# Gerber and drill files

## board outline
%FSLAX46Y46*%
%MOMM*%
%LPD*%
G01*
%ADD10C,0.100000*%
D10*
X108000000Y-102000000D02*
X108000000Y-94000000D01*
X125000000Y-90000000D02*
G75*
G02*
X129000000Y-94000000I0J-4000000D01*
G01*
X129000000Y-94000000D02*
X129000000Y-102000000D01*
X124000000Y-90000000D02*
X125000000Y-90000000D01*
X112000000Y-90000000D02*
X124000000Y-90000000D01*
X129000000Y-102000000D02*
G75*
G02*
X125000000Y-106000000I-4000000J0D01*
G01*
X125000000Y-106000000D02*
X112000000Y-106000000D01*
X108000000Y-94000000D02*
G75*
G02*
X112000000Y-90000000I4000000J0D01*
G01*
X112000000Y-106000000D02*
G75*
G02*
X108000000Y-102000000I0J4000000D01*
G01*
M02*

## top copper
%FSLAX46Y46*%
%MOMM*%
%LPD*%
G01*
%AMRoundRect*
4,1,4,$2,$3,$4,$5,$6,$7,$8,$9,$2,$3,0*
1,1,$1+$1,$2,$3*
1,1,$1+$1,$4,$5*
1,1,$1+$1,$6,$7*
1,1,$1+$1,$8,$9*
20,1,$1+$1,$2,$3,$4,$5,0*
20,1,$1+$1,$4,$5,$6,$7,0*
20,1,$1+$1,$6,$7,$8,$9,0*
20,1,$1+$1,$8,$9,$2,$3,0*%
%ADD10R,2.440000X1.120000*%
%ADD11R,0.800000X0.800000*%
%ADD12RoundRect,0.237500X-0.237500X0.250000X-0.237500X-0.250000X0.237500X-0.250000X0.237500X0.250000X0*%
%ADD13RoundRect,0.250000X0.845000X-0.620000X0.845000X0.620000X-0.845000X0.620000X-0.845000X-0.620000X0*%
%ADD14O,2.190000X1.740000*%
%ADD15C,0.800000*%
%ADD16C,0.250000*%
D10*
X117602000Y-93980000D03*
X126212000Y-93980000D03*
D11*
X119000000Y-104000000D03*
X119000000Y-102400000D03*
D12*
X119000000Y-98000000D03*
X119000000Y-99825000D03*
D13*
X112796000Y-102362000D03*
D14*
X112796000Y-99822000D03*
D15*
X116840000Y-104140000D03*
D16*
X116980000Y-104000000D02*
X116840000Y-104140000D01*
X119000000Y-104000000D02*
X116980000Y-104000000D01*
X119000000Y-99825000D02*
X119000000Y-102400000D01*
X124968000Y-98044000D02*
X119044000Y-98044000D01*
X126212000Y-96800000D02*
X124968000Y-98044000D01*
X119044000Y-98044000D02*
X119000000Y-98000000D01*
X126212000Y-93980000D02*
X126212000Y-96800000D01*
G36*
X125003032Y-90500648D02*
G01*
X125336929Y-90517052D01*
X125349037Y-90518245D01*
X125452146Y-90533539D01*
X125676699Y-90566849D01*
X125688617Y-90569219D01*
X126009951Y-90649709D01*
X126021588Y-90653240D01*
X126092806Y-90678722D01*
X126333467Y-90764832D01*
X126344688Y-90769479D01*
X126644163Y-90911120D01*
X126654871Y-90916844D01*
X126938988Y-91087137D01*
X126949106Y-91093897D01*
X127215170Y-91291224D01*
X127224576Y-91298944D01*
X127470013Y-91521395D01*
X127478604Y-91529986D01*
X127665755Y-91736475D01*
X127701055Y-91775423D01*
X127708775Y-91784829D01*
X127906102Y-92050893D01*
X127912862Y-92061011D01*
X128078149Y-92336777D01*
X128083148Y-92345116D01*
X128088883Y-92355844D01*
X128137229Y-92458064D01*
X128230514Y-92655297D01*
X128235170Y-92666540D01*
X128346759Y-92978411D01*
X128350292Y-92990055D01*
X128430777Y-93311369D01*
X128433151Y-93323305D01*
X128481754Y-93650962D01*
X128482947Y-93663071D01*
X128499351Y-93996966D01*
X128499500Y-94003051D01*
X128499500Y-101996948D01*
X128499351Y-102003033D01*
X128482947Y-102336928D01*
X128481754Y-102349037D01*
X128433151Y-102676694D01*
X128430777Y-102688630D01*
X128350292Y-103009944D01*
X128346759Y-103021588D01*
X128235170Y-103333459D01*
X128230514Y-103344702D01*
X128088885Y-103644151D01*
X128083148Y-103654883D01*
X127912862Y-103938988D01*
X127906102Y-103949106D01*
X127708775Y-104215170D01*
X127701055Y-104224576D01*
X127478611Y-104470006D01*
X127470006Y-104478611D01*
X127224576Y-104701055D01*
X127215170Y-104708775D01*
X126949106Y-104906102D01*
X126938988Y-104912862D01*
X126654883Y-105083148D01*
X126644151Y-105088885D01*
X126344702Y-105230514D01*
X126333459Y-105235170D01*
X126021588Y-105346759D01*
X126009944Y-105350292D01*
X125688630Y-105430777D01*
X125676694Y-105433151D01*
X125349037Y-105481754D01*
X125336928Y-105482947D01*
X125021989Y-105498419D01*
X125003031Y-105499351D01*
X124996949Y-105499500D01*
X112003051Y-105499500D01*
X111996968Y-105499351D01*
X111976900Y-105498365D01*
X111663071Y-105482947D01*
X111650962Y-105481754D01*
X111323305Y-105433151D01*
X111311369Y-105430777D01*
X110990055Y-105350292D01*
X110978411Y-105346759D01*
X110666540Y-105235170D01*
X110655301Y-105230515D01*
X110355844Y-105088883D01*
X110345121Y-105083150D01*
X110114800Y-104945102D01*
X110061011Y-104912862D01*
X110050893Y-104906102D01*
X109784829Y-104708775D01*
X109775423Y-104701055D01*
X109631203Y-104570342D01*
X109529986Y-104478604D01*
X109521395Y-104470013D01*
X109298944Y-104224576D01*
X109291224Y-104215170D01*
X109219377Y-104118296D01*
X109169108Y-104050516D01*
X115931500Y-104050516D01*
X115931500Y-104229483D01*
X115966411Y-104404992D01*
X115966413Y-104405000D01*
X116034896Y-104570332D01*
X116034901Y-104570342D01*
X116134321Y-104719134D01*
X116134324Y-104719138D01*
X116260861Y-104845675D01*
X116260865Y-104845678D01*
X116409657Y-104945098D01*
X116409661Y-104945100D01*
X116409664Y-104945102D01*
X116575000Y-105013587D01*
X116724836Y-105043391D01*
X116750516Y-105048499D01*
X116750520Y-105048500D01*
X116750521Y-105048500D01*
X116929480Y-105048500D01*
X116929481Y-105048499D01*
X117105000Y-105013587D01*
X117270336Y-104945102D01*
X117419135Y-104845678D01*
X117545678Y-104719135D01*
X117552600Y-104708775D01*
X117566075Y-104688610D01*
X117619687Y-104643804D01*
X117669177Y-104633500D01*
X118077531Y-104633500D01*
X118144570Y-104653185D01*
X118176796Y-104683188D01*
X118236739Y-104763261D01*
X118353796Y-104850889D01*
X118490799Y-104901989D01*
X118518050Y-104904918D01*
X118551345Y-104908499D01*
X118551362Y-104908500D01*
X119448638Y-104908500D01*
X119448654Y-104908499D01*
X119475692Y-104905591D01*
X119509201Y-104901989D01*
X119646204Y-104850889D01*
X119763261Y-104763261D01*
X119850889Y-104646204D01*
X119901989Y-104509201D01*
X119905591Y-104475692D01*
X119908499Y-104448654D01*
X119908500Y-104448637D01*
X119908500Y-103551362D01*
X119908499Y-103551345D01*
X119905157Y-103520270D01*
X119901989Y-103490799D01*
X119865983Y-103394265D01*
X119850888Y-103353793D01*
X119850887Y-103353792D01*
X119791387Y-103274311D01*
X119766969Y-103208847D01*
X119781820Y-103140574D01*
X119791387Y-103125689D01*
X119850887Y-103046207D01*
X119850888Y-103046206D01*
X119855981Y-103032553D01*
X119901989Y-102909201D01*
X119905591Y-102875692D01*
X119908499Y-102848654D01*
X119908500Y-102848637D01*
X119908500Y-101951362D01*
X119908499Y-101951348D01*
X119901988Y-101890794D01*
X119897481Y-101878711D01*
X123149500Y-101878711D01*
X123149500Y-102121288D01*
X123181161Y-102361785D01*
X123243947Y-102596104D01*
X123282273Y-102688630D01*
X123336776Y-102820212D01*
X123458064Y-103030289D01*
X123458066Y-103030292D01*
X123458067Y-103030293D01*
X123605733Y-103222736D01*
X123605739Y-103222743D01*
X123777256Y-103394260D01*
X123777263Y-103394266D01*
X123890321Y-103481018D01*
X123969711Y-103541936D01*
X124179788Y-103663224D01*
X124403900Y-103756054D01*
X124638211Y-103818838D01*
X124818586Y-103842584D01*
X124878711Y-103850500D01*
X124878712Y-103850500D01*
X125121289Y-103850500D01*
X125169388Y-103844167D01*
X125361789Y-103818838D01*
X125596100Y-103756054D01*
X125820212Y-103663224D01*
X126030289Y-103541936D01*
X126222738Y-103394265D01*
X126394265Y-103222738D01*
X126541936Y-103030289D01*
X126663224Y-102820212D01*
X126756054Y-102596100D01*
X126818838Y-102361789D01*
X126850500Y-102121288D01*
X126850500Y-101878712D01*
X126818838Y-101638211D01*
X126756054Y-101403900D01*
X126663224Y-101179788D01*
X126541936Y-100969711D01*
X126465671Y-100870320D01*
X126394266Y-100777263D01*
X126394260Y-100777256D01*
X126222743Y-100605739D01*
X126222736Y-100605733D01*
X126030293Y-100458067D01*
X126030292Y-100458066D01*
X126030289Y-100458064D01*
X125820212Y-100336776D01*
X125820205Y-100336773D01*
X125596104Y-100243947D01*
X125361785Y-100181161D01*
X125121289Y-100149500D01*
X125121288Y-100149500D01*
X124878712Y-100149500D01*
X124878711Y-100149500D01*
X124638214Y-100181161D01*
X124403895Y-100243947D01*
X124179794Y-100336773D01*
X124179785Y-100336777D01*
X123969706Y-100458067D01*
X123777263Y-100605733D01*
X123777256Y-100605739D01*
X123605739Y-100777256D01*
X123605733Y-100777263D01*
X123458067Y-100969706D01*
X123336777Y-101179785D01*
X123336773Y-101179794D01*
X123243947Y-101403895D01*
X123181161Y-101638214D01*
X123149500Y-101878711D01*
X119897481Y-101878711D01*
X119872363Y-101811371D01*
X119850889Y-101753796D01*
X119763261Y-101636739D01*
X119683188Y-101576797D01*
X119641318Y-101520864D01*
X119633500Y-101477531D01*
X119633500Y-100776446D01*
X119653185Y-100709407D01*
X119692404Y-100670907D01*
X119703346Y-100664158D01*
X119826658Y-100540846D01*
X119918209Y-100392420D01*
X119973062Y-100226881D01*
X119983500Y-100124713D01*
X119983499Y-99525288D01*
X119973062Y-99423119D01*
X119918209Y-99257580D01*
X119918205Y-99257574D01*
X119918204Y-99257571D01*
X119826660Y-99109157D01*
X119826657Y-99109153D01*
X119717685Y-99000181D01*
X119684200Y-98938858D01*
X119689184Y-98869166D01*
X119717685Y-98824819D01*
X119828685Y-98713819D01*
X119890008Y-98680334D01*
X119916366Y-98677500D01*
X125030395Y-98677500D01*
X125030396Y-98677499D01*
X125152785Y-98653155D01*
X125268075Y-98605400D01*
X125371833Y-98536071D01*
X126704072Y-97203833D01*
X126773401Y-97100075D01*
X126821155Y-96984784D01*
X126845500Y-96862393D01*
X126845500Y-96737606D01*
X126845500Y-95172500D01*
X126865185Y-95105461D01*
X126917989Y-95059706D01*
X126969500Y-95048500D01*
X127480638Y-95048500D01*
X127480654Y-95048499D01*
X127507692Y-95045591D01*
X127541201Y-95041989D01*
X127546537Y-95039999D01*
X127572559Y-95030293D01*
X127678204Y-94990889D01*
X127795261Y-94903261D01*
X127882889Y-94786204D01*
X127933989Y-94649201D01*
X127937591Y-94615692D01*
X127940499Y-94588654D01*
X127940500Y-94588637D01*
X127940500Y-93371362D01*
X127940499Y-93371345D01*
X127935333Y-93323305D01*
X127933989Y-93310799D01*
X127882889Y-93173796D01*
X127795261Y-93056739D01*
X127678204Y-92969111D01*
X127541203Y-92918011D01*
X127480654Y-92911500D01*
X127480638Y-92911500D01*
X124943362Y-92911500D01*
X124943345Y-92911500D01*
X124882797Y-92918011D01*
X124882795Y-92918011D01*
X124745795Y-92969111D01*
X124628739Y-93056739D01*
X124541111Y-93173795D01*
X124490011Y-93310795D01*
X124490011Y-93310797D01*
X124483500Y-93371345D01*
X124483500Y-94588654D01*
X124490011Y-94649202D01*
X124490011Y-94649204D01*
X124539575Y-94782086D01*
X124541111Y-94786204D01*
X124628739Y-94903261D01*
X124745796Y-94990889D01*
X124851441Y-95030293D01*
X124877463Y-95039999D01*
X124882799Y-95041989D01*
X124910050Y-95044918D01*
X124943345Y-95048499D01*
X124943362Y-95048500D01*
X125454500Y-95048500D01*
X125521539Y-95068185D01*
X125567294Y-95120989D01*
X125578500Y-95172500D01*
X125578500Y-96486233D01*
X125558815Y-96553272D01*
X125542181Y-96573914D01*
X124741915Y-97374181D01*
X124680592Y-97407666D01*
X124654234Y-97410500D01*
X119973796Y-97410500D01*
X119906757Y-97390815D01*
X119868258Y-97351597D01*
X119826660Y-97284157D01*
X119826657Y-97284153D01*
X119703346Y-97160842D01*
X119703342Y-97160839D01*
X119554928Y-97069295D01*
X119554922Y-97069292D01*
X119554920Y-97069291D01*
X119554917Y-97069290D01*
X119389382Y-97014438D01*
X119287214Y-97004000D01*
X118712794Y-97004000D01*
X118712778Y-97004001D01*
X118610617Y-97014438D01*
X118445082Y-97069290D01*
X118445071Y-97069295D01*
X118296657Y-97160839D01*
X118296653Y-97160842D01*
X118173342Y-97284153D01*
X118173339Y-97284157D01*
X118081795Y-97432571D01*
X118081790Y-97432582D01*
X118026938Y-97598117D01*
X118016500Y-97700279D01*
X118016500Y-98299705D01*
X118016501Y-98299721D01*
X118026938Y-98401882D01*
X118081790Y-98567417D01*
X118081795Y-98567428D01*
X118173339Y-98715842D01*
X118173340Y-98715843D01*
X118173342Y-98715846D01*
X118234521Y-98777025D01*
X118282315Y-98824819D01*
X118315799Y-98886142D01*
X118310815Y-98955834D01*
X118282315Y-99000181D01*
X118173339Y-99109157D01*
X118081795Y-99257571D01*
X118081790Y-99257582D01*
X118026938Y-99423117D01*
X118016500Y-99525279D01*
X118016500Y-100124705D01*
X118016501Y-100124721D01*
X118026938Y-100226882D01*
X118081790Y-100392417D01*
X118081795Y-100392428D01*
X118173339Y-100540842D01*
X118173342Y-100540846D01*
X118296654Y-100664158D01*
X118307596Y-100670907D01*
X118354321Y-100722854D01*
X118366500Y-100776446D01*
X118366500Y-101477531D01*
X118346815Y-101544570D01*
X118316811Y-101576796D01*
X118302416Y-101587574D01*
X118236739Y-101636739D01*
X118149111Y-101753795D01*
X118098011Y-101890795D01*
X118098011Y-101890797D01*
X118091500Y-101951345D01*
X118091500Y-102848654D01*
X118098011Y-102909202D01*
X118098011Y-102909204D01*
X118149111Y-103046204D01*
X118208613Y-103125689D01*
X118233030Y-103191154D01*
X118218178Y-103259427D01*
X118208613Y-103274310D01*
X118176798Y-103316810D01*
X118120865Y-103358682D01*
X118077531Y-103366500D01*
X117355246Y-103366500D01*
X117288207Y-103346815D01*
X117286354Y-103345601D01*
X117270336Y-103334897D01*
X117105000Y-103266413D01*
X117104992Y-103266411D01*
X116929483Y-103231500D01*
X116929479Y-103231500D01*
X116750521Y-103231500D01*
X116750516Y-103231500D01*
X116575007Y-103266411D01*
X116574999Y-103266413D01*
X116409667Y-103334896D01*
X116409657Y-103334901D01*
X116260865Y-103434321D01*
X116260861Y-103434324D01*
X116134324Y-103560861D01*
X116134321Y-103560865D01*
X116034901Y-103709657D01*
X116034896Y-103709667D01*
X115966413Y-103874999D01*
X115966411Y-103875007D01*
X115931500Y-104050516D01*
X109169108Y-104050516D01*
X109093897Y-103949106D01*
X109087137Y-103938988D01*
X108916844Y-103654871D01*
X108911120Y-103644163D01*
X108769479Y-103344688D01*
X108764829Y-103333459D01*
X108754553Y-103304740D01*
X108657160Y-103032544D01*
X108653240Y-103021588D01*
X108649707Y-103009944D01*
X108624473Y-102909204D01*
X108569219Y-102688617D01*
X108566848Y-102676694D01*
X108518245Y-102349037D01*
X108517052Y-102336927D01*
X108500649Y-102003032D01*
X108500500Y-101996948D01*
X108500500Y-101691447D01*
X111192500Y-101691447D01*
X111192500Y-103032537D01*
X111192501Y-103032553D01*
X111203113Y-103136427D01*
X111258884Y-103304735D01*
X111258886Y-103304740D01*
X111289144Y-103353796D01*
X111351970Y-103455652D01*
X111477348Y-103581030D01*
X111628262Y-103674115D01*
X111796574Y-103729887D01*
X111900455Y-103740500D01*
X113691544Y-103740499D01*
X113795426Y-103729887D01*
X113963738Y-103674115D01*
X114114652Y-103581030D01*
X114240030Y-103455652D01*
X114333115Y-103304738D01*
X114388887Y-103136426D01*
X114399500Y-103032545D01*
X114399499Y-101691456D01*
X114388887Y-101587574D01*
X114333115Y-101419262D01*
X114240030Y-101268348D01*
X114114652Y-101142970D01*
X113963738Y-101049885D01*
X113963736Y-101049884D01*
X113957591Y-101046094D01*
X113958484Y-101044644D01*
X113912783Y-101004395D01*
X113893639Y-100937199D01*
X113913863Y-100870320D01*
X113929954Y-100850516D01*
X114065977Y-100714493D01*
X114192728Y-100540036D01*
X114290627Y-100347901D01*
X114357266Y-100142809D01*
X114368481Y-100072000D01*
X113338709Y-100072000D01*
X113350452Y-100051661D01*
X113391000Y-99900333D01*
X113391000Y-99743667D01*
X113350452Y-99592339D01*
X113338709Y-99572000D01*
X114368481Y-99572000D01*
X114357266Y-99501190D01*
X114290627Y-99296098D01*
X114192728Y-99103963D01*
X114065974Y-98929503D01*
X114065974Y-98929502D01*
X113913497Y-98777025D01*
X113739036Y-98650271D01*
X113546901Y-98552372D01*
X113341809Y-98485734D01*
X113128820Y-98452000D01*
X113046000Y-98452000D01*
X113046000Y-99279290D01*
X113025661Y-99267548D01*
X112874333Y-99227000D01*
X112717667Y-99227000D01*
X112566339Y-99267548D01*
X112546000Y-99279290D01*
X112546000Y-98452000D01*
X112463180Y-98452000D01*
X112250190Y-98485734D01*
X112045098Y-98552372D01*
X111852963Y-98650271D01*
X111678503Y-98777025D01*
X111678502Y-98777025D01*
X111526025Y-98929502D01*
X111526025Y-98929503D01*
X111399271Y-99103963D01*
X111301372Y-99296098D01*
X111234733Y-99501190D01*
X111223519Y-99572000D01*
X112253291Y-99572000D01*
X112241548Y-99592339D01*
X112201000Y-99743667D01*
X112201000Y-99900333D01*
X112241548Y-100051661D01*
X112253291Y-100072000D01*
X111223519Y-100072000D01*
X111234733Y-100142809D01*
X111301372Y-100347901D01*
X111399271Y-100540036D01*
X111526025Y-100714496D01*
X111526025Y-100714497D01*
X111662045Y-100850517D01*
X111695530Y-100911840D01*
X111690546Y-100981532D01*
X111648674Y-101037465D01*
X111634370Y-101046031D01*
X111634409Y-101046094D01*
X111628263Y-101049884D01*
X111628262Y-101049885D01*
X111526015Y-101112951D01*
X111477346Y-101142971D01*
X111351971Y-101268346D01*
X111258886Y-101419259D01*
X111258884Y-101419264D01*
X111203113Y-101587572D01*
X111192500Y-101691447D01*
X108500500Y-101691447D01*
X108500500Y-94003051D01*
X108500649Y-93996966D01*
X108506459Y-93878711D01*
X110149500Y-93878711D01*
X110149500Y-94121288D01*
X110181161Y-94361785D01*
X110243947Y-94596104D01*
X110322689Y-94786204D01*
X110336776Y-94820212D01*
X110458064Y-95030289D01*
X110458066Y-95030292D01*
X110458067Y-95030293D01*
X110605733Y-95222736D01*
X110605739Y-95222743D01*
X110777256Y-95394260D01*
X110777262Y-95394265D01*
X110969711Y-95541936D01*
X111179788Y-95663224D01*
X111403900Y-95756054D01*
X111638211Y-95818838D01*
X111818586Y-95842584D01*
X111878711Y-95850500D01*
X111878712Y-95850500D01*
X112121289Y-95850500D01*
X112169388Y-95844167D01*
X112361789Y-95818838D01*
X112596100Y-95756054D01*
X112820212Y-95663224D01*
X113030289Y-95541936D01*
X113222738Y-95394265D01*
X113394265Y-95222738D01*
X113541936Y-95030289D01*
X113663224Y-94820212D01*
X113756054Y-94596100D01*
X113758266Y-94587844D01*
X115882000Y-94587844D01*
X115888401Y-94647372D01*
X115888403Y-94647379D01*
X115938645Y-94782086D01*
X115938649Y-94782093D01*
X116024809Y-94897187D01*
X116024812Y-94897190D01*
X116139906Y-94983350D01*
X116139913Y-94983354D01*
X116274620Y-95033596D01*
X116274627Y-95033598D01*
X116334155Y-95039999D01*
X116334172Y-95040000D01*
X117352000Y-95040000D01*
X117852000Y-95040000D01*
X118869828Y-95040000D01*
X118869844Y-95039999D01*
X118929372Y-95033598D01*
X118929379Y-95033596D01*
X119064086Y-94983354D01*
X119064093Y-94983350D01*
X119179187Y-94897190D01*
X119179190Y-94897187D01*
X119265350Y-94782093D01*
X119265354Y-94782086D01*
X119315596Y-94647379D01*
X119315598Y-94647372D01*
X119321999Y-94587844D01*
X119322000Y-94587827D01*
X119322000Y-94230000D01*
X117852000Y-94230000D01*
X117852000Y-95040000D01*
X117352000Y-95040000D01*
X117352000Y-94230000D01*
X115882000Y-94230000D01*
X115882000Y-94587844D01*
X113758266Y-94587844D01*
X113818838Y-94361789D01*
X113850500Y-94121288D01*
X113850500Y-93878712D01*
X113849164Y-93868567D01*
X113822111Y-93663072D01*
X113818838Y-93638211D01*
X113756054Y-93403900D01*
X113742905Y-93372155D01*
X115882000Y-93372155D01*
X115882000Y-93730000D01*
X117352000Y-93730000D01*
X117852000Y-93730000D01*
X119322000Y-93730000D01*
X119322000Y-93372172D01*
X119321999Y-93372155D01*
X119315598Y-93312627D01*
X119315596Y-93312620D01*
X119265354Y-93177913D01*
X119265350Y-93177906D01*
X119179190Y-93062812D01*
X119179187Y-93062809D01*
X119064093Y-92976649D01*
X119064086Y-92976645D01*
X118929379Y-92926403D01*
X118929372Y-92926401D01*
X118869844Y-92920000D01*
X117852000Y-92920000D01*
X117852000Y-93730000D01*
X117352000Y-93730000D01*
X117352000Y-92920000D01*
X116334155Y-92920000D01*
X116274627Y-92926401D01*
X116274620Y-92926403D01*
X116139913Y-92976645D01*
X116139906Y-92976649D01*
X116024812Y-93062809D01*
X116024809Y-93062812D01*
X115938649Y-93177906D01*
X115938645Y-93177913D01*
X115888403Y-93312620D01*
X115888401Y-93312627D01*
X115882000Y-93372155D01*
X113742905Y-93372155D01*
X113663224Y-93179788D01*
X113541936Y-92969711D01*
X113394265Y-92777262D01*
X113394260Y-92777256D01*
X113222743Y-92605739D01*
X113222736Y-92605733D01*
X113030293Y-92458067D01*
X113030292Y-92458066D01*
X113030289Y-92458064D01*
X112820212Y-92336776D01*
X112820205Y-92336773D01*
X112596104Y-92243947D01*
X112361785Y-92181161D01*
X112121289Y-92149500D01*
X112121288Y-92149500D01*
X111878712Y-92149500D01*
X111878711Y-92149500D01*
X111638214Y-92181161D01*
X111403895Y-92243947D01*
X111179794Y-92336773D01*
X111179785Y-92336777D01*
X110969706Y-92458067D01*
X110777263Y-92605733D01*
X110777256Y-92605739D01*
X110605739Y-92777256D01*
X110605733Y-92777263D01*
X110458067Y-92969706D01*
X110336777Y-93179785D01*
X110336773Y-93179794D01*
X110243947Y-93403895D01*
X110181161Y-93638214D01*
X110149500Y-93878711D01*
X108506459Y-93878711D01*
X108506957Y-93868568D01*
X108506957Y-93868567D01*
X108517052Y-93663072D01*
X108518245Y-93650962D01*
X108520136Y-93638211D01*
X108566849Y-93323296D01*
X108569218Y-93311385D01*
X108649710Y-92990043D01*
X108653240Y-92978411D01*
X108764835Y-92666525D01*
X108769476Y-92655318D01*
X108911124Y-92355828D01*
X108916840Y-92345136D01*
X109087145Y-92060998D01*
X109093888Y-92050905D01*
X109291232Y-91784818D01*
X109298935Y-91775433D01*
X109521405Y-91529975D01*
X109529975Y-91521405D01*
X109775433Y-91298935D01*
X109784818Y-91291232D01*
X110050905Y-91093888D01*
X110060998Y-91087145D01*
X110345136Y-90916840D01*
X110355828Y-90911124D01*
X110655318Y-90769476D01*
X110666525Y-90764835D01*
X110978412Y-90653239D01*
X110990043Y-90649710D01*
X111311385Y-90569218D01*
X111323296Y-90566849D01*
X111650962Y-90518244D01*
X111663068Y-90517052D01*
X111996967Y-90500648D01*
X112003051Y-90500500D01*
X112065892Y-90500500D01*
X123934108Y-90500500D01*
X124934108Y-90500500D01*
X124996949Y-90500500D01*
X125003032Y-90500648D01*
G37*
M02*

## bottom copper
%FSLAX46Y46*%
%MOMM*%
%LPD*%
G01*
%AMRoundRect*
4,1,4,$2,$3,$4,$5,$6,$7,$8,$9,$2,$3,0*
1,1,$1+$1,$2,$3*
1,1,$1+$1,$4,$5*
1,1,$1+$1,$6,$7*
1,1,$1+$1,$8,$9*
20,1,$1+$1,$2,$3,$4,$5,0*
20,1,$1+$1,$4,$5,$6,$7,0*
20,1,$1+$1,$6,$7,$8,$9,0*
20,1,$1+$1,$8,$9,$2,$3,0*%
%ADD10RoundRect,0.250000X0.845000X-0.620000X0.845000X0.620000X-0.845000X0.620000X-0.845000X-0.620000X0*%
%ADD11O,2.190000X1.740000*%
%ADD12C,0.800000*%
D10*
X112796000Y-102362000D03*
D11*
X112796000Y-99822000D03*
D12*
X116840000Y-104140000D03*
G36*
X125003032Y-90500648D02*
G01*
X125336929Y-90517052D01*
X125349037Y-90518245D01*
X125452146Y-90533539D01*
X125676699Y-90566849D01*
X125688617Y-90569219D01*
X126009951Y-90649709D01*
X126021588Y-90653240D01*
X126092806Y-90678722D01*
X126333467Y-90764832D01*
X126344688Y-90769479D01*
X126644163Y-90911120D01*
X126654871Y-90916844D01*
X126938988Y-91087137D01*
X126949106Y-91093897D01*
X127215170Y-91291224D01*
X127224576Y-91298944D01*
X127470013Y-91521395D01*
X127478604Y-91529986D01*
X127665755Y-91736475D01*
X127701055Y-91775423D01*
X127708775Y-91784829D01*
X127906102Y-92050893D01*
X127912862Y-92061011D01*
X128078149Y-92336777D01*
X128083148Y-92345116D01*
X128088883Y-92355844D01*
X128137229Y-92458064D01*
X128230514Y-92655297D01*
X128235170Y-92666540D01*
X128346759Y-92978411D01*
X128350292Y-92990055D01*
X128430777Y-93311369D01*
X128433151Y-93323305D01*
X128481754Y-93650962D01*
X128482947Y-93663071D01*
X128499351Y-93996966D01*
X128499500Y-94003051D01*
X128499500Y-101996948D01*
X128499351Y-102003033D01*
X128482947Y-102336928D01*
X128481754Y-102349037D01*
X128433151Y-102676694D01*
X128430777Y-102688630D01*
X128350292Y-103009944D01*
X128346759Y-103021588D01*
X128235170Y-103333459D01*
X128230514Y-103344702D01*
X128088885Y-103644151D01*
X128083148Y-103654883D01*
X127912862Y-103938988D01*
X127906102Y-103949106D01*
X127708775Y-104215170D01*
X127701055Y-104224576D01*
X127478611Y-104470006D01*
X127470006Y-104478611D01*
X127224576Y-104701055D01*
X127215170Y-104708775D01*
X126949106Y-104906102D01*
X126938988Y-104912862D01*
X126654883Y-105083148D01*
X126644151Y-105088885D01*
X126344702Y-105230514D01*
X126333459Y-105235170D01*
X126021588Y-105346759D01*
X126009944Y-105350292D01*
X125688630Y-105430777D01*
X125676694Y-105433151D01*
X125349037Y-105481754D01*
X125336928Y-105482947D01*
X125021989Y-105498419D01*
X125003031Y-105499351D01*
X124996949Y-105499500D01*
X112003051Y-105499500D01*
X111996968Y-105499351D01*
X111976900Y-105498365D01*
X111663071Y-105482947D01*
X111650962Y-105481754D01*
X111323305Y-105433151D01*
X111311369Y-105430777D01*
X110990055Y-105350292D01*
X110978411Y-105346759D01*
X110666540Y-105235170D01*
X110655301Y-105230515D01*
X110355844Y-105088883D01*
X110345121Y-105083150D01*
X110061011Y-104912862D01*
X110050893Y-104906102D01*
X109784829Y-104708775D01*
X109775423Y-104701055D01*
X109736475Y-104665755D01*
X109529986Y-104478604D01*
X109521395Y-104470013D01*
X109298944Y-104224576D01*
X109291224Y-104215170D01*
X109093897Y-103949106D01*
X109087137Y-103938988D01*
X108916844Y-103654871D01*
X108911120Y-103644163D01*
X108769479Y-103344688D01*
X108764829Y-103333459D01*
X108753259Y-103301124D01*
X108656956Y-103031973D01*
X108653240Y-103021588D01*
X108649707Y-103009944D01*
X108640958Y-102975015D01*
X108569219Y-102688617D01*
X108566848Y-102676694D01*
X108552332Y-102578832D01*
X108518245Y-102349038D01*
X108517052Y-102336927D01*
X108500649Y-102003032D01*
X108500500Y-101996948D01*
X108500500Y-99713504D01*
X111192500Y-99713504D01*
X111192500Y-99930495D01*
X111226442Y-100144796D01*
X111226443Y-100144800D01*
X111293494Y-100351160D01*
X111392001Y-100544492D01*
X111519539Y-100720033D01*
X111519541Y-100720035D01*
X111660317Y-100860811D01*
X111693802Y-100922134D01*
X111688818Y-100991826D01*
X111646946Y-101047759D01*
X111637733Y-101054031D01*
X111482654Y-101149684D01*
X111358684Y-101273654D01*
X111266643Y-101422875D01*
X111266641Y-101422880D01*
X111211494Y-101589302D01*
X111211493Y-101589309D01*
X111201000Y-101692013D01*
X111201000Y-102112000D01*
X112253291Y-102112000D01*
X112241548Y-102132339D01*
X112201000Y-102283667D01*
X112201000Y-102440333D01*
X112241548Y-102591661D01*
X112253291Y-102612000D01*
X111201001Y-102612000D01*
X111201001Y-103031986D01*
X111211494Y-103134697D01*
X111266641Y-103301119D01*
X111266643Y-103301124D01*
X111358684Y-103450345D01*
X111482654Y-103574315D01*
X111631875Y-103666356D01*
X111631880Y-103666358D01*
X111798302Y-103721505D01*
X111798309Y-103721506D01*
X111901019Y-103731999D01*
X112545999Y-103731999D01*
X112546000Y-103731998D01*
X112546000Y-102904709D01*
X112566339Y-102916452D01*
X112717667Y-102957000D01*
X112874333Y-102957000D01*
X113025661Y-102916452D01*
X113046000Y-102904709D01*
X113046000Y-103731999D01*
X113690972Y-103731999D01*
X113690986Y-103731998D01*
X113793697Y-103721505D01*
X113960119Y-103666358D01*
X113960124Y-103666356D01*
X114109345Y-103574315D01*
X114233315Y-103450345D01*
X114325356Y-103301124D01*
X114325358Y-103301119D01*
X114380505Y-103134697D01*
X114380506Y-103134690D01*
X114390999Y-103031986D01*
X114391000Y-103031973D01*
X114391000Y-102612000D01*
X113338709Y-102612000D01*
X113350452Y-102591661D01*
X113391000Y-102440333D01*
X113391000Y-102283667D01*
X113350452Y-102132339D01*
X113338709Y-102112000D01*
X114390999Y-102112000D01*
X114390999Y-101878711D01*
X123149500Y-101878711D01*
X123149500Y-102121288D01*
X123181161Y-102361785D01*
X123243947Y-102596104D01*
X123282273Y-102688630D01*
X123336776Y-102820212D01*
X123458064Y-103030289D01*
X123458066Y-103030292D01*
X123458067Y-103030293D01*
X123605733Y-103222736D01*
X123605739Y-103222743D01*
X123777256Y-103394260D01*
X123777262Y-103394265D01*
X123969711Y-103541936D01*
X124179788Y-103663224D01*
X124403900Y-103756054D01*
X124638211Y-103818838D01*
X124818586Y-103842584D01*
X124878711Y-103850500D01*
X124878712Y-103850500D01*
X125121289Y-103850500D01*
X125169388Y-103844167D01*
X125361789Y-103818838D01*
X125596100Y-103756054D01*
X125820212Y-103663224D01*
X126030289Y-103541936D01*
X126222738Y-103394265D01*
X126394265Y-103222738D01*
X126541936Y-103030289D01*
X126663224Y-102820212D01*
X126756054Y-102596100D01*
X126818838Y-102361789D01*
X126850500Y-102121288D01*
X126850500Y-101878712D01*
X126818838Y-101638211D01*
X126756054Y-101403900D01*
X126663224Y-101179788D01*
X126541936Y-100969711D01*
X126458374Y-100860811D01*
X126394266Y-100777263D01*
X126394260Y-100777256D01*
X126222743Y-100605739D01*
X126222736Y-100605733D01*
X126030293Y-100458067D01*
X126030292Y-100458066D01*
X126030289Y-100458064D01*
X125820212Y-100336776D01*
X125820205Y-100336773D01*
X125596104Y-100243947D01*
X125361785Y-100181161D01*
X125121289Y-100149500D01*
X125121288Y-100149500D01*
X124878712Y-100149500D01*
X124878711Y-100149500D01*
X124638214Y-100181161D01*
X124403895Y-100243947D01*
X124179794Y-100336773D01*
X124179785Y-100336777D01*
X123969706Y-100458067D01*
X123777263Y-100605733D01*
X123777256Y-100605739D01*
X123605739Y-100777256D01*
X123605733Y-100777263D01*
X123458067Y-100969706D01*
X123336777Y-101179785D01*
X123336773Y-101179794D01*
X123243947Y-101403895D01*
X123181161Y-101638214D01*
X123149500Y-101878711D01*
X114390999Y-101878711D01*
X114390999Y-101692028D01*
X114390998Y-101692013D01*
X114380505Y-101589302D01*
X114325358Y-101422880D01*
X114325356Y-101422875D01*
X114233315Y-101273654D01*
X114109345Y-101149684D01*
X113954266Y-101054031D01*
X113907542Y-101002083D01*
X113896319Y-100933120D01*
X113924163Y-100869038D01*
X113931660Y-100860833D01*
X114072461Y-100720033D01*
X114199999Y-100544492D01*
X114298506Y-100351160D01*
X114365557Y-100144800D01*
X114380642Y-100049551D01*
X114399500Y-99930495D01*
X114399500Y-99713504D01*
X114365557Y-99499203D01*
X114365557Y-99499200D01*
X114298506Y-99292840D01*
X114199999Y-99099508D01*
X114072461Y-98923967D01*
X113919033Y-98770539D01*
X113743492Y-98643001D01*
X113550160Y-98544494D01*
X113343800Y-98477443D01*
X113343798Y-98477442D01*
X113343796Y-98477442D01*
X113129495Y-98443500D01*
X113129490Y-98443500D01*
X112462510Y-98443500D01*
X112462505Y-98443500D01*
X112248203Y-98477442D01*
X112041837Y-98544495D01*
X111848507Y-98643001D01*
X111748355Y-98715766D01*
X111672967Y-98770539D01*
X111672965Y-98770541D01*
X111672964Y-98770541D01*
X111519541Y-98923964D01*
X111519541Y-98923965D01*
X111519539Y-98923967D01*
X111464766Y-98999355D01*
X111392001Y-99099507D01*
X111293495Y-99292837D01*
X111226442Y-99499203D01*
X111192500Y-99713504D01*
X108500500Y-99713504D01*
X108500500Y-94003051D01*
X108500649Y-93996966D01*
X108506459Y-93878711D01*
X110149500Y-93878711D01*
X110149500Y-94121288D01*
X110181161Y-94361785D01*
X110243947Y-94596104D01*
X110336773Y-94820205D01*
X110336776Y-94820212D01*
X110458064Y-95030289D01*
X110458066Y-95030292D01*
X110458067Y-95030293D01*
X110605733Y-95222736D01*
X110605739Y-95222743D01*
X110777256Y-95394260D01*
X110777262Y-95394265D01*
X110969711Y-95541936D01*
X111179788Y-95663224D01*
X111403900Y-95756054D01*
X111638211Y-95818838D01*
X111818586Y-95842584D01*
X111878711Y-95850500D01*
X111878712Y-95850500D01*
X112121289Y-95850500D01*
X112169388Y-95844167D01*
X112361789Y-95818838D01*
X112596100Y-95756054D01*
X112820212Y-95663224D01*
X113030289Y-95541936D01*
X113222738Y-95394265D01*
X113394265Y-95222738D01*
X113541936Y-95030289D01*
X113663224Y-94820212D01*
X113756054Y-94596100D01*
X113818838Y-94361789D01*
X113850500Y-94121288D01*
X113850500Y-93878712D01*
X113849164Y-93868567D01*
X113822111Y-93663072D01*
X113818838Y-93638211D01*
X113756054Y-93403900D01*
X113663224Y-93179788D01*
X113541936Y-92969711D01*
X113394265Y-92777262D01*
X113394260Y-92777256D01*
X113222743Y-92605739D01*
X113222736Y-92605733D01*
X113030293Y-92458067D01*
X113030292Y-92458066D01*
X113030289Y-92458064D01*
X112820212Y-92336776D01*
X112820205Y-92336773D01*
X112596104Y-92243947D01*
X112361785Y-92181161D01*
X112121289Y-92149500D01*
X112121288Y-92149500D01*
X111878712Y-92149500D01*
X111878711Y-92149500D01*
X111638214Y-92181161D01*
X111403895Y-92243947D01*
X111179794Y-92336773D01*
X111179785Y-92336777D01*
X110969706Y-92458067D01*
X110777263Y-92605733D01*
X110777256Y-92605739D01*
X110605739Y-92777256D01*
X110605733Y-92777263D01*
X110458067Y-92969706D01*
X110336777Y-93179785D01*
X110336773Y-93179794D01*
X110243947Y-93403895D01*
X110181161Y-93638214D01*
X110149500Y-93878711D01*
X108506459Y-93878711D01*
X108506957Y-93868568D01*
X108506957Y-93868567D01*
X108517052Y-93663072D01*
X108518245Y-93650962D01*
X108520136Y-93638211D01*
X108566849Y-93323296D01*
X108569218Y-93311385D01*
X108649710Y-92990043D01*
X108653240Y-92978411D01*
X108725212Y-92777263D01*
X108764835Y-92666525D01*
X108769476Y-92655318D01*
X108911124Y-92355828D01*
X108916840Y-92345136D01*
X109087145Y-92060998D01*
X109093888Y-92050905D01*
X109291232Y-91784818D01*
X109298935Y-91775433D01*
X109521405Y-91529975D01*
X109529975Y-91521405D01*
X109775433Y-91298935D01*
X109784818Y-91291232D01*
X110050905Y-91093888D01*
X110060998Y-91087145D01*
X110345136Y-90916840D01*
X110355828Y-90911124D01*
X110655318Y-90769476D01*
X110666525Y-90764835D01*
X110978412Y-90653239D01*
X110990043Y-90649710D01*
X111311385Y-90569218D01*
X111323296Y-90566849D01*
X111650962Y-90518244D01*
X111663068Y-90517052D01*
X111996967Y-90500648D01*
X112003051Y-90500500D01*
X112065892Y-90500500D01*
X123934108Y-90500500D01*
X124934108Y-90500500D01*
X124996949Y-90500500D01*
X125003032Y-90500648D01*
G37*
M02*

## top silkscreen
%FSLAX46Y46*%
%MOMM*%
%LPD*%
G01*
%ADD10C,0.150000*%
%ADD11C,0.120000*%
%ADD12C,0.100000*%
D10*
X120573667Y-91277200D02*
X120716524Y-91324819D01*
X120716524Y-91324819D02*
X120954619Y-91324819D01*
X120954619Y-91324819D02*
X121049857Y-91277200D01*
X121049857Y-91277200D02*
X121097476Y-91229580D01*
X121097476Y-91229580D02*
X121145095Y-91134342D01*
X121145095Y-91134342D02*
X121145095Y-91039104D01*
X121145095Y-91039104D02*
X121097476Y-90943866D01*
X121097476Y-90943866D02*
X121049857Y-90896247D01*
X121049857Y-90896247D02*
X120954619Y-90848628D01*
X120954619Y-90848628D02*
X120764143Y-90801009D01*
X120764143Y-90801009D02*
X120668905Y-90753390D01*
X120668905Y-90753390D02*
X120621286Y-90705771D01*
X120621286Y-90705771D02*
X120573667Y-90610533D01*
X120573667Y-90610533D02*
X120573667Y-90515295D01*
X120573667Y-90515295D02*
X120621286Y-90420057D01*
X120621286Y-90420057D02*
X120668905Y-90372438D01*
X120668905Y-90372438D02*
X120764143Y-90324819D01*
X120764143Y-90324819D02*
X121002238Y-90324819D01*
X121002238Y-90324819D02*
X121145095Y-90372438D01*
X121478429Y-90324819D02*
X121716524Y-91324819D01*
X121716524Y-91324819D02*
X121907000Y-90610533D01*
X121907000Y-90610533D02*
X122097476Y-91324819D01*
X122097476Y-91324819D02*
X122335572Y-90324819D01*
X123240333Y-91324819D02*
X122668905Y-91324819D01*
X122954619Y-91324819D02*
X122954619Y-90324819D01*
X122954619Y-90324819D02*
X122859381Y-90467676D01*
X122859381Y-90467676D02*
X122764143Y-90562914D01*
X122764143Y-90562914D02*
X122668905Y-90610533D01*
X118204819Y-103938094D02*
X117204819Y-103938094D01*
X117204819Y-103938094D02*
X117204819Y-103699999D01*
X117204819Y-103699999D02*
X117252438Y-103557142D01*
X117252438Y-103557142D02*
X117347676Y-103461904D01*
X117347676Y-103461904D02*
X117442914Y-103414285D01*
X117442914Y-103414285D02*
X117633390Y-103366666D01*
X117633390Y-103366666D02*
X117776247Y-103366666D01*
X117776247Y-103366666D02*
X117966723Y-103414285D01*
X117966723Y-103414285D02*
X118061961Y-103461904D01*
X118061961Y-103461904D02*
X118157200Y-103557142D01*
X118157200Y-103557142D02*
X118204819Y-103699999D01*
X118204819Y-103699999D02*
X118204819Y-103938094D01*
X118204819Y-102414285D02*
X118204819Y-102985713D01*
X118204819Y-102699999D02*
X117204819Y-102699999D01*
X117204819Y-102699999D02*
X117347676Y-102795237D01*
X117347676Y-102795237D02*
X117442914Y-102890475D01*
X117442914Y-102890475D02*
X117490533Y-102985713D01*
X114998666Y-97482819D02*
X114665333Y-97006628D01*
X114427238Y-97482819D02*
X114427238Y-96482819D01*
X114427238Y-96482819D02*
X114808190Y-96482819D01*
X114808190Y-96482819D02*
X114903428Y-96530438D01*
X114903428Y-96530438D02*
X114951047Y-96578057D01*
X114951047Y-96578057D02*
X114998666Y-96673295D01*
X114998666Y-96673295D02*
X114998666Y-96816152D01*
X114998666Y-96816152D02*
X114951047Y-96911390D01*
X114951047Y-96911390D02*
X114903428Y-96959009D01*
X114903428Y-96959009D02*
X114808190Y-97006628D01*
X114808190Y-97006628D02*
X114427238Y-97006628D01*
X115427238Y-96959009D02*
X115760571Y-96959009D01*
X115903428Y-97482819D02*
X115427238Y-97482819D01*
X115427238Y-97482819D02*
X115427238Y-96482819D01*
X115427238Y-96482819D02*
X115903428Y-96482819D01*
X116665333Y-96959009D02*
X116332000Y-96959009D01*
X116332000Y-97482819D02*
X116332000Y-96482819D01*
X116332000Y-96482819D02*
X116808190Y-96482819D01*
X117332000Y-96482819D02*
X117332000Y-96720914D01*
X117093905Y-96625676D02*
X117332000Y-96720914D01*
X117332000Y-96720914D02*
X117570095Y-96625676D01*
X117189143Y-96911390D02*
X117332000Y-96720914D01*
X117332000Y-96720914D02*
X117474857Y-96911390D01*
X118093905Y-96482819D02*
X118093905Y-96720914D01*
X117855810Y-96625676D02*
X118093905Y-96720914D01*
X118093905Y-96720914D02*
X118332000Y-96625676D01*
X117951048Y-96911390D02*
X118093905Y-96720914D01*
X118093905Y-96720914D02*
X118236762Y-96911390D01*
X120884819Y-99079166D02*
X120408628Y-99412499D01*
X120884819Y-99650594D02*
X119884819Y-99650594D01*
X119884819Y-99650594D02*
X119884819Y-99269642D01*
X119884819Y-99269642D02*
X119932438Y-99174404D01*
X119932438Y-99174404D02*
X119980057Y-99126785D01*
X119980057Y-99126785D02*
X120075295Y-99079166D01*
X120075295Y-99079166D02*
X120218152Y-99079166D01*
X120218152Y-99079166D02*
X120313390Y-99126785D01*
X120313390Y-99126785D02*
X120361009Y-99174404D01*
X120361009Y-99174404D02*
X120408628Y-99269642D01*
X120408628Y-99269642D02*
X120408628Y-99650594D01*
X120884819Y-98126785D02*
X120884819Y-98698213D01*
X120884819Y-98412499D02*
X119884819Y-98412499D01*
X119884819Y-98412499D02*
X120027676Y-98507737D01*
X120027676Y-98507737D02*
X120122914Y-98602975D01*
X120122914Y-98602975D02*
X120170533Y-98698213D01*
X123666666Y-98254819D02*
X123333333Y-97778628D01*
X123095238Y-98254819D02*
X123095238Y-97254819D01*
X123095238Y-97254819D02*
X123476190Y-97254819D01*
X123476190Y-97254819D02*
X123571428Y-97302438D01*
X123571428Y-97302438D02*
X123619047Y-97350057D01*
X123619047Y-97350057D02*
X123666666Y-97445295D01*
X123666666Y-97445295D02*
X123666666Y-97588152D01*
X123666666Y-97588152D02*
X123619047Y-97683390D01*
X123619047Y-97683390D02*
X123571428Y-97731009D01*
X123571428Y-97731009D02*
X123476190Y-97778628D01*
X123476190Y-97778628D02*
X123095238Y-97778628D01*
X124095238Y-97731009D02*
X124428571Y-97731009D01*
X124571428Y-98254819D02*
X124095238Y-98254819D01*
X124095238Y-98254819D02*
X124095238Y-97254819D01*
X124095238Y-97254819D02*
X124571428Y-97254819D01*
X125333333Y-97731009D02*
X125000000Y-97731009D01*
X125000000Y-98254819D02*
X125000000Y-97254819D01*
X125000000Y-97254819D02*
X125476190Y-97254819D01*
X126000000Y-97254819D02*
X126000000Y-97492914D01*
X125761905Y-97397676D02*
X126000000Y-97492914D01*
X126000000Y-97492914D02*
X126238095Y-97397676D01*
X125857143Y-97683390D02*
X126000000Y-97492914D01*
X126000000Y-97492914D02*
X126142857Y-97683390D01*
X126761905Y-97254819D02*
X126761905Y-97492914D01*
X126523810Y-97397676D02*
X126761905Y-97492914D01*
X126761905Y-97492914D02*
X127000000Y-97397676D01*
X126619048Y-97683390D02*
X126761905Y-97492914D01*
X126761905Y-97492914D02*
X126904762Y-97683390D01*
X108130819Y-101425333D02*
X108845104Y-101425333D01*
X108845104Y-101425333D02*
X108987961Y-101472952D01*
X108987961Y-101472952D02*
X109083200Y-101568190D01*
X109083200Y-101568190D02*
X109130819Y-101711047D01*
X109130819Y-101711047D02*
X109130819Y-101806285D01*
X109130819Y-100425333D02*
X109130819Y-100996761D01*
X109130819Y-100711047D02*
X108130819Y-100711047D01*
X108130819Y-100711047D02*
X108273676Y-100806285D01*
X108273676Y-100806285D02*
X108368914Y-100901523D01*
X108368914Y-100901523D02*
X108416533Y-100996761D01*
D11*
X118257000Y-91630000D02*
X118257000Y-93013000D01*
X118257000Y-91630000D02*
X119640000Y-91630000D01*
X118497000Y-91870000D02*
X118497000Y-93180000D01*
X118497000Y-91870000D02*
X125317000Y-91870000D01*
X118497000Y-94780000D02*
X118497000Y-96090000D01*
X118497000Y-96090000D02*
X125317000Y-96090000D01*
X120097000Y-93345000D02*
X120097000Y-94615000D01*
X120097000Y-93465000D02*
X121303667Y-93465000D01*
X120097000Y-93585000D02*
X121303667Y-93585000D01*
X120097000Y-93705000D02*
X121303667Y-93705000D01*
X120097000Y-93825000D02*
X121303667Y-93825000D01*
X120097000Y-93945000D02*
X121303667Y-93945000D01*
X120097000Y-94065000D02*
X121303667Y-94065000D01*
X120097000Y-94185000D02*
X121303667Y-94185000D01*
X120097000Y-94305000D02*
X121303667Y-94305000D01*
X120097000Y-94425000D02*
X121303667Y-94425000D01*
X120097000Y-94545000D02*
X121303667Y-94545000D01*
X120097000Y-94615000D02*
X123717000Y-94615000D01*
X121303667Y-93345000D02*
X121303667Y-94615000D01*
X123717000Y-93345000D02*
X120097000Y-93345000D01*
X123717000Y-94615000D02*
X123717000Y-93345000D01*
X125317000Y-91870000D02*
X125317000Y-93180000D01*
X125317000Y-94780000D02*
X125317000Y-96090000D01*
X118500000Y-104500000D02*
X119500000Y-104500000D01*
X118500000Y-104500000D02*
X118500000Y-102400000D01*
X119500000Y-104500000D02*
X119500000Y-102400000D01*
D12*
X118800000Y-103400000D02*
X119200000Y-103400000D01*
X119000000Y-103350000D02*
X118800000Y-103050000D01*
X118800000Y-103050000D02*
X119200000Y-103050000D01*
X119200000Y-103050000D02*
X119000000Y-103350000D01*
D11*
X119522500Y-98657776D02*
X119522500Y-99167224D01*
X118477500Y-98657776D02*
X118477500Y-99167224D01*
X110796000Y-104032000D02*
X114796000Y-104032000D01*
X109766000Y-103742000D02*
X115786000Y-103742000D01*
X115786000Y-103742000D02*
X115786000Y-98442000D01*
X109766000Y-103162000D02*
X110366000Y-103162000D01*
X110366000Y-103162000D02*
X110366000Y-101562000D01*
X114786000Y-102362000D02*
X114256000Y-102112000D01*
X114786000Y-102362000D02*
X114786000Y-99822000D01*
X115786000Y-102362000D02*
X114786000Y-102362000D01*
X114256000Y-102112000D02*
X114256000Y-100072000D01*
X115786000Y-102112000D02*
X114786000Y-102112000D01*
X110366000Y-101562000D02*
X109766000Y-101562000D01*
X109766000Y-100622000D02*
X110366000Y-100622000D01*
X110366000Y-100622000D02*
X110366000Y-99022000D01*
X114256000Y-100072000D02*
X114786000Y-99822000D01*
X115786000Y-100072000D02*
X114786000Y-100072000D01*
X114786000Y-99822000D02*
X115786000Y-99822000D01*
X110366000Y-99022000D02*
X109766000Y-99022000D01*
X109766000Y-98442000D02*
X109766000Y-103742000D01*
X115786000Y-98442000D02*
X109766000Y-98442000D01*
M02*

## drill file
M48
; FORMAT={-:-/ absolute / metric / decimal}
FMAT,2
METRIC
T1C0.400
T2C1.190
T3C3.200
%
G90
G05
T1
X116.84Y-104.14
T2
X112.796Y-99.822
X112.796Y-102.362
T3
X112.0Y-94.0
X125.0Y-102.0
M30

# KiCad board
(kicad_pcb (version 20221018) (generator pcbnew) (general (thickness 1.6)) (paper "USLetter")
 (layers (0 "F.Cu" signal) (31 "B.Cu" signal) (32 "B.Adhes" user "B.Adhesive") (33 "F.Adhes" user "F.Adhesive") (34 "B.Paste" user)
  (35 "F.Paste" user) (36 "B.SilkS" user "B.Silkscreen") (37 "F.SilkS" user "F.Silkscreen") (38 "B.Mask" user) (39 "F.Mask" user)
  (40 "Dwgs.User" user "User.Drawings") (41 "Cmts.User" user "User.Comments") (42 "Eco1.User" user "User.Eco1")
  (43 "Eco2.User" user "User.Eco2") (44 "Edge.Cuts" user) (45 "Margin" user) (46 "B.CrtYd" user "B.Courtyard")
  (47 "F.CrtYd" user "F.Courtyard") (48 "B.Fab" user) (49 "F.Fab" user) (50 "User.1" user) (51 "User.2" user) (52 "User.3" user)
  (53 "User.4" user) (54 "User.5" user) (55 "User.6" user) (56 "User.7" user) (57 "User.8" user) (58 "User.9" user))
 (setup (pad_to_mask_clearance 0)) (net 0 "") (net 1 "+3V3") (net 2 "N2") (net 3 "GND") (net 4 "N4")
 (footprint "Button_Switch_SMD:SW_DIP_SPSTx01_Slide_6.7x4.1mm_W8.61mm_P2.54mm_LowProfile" (layer "F.Cu") (at 121.907 93.98)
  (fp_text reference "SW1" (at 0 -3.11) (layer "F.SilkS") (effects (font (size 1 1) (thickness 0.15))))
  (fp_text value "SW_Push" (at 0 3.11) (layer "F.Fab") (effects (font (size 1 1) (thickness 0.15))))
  (fp_line (start -3.65 -2.35) (end -3.65 -0.967) (stroke (width 0.12) (type solid)) (layer "F.SilkS"))
  (fp_line (start -3.65 -2.35) (end -2.267 -2.35) (stroke (width 0.12) (type solid)) (layer "F.SilkS"))
  (fp_line (start -3.41 -2.11) (end -3.41 -0.8) (stroke (width 0.12) (type solid)) (layer "F.SilkS"))
  (fp_line (start -3.41 -2.11) (end 3.41 -2.11) (stroke (width 0.12) (type solid)) (layer "F.SilkS"))
  (fp_line (start -3.41 0.8) (end -3.41 2.11) (stroke (width 0.12) (type solid)) (layer "F.SilkS"))
  (fp_line (start -3.41 2.11) (end 3.41 2.11) (stroke (width 0.12) (type solid)) (layer "F.SilkS"))
  (fp_line (start -1.81 -0.635) (end -1.81 0.635) (stroke (width 0.12) (type solid)) (layer "F.SilkS"))
  (fp_line (start -1.81 -0.515) (end -0.603333 -0.515) (stroke (width 0.12) (type solid)) (layer "F.SilkS"))
  (fp_line (start -1.81 -0.395) (end -0.603333 -0.395) (stroke (width 0.12) (type solid)) (layer "F.SilkS"))
  (fp_line (start -1.81 -0.275) (end -0.603333 -0.275) (stroke (width 0.12) (type solid)) (layer "F.SilkS"))
  (fp_line (start -1.81 -0.155) (end -0.603333 -0.155) (stroke (width 0.12) (type solid)) (layer "F.SilkS"))
  (fp_line (start -1.81 -0.035) (end -0.603333 -0.035) (stroke (width 0.12) (type solid)) (layer "F.SilkS"))
  (fp_line (start -1.81 0.085) (end -0.603333 0.085) (stroke (width 0.12) (type solid)) (layer "F.SilkS"))
  (fp_line (start -1.81 0.205) (end -0.603333 0.205) (stroke (width 0.12) (type solid)) (layer "F.SilkS"))
  (fp_line (start -1.81 0.325) (end -0.603333 0.325) (stroke (width 0.12) (type solid)) (layer "F.SilkS"))
  (fp_line (start -1.81 0.445) (end -0.603333 0.445) (stroke (width 0.12) (type solid)) (layer "F.SilkS"))
  (fp_line (start -1.81 0.565) (end -0.603333 0.565) (stroke (width 0.12) (type solid)) (layer "F.SilkS"))
  (fp_line (start -1.81 0.635) (end 1.81 0.635) (stroke (width 0.12) (type solid)) (layer "F.SilkS"))
  (fp_line (start -0.603333 -0.635) (end -0.603333 0.635) (stroke (width 0.12) (type solid)) (layer "F.SilkS"))
  (fp_line (start 1.81 -0.635) (end -1.81 -0.635) (stroke (width 0.12) (type solid)) (layer "F.SilkS"))
  (fp_line (start 1.81 0.635) (end 1.81 -0.635) (stroke (width 0.12) (type solid)) (layer "F.SilkS"))
  (fp_line (start 3.41 -2.11) (end 3.41 -0.8) (stroke (width 0.12) (type solid)) (layer "F.SilkS"))
  (fp_line (start 3.41 0.8) (end 3.41 2.11) (stroke (width 0.12) (type solid)) (layer "F.SilkS"))
  (pad "1" smd rect (at -4.305 0) (size 2.44 1.12) (layers "F.Cu" "F.Paste" "F.Mask") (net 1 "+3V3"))
  (pad "2" smd rect (at 4.305 0) (size 2.44 1.12) (layers "F.Cu" "F.Paste" "F.Mask") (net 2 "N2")))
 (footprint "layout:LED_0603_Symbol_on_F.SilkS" (layer "F.Cu") (at 119 103.2 90)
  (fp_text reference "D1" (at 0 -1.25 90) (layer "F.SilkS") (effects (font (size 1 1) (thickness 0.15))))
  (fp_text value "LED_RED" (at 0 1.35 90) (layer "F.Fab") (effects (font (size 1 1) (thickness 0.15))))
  (fp_line (start -1.3 -0.5) (end -1.3 0.5) (stroke (width 0.12) (type solid)) (layer "F.SilkS"))
  (fp_line (start -1.3 -0.5) (end 0.8 -0.5) (stroke (width 0.12) (type solid)) (layer "F.SilkS"))
  (fp_line (start -1.3 0.5) (end 0.8 0.5) (stroke (width 0.12) (type solid)) (layer "F.SilkS"))
  (fp_line (start -0.2 -0.2) (end -0.2 0.2) (stroke (width 0.1) (type solid)) (layer "F.SilkS"))
  (fp_line (start -0.15 0) (end 0.15 -0.2) (stroke (width 0.1) (type solid)) (layer "F.SilkS"))
  (fp_line (start 0.15 -0.2) (end 0.15 0.2) (stroke (width 0.1) (type solid)) (layer "F.SilkS"))
  (fp_line (start 0.15 0.2) (end -0.15 0) (stroke (width 0.1) (type solid)) (layer "F.SilkS"))
  (pad "1" smd rect (at -0.8 0 270) (size 0.8 0.8) (layers "F.Cu" "F.Paste" "F.Mask") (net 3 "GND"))
  (pad "2" smd rect (at 0.8 0 270) (size 0.8 0.8) (layers "F.Cu" "F.Paste" "F.Mask") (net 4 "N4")))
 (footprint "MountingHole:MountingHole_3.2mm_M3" (layer "F.Cu") (at 112 94)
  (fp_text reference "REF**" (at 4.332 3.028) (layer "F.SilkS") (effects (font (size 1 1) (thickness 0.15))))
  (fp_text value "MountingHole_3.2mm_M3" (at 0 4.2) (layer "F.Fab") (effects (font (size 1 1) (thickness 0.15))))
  (pad "" np_thru_hole circle (at 0 0) (size 3.2 3.2) (drill 3.2) (layers "*.Cu" "*.Mask")))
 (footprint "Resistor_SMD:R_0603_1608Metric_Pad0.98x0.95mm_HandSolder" (layer "F.Cu") (at 119 98.9125 -90)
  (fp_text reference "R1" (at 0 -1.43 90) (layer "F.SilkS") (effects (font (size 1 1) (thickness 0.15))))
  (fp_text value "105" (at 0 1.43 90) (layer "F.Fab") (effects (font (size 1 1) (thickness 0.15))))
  (fp_line (start -0.254724 -0.5225) (end 0.254724 -0.5225) (stroke (width 0.12) (type solid)) (layer "F.SilkS"))
  (fp_line (start -0.254724 0.5225) (end 0.254724 0.5225) (stroke (width 0.12) (type solid)) (layer "F.SilkS"))
  (pad "1" smd roundrect (at -0.9125 0 270) (size 0.975 0.95) (layers "F.Cu" "F.Paste" "F.Mask") (roundrect_rratio 0.25) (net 2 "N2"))
  (pad "2" smd roundrect (at 0.9125 0 270) (size 0.975 0.95) (layers "F.Cu" "F.Paste" "F.Mask") (roundrect_rratio 0.25) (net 4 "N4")))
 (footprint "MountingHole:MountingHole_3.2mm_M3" (layer "F.Cu") (at 125 102)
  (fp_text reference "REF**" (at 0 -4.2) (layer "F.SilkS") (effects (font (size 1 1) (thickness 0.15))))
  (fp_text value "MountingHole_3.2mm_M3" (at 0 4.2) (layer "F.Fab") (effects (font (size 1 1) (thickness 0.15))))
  (pad "" np_thru_hole circle (at 0 0) (size 3.2 3.2) (drill 3.2) (layers "*.Cu" "*.Mask")))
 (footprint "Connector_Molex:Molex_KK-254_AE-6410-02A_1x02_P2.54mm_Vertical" (layer "F.Cu") (at 112.796 102.362 90)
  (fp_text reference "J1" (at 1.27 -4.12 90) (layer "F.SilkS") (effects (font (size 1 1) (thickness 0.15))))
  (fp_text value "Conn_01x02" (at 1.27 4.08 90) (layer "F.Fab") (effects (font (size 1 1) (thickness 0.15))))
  (fp_line (start -1.67 -2) (end -1.67 2) (stroke (width 0.12) (type solid)) (layer "F.SilkS"))
  (fp_line (start -1.38 -3.03) (end -1.38 2.99) (stroke (width 0.12) (type solid)) (layer "F.SilkS"))
  (fp_line (start -1.38 2.99) (end 3.92 2.99) (stroke (width 0.12) (type solid)) (layer "F.SilkS"))
  (fp_line (start -0.8 -3.03) (end -0.8 -2.43) (stroke (width 0.12) (type solid)) (layer "F.SilkS"))
  (fp_line (start -0.8 -2.43) (end 0.8 -2.43) (stroke (width 0.12) (type solid)) (layer "F.SilkS"))
  (fp_line (start 0 1.99) (end 0.25 1.46) (stroke (width 0.12) (type solid)) (layer "F.SilkS"))
  (fp_line (start 0 1.99) (end 2.54 1.99) (stroke (width 0.12) (type solid)) (layer "F.SilkS"))
  (fp_line (start 0 2.99) (end 0 1.99) (stroke (width 0.12) (type solid)) (layer "F.SilkS"))
  (fp_line (start 0.25 1.46) (end 2.29 1.46) (stroke (width 0.12) (type solid)) (layer "F.SilkS"))
  (fp_line (start 0.25 2.99) (end 0.25 1.99) (stroke (width 0.12) (type solid)) (layer "F.SilkS"))
  (fp_line (start 0.8 -2.43) (end 0.8 -3.03) (stroke (width 0.12) (type solid)) (layer "F.SilkS"))
  (fp_line (start 1.74 -3.03) (end 1.74 -2.43) (stroke (width 0.12) (type solid)) (layer "F.SilkS"))
  (fp_line (start 1.74 -2.43) (end 3.34 -2.43) (stroke (width 0.12) (type solid)) (layer "F.SilkS"))
  (fp_line (start 2.29 1.46) (end 2.54 1.99) (stroke (width 0.12) (type solid)) (layer "F.SilkS"))
  (fp_line (start 2.29 2.99) (end 2.29 1.99) (stroke (width 0.12) (type solid)) (layer "F.SilkS"))
  (fp_line (start 2.54 1.99) (end 2.54 2.99) (stroke (width 0.12) (type solid)) (layer "F.SilkS"))
  (fp_line (start 3.34 -2.43) (end 3.34 -3.03) (stroke (width 0.12) (type solid)) (layer "F.SilkS"))
  (fp_line (start 3.92 -3.03) (end -1.38 -3.03) (stroke (width 0.12) (type solid)) (layer "F.SilkS"))
  (fp_line (start 3.92 2.99) (end 3.92 -3.03) (stroke (width 0.12) (type solid)) (layer "F.SilkS"))
  (pad "1" thru_hole roundrect (at 0 0 90) (size 1.74 2.19) (drill 1.19) (layers "*.Cu" "*.Mask") (roundrect_rratio 0.143678) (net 3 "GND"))
  (pad "2" thru_hole oval (at 2.54 0 90) (size 1.74 2.19) (drill 1.19) (layers "*.Cu" "*.Mask") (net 1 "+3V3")))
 (gr_line (start 108 102) (end 108 94) (stroke (width 0.1) (type default)) (layer "Edge.Cuts"))
 (gr_arc (start 125 90) (mid 127.828427 91.171573) (end 129 94) (stroke (width 0.1) (type default)) (layer "Edge.Cuts"))
 (gr_line (start 129 94) (end 129 102) (stroke (width 0.1) (type default)) (layer "Edge.Cuts"))
 (gr_line (start 124 90) (end 125 90) (stroke (width 0.1) (type default)) (layer "Edge.Cuts"))
 (gr_line (start 112 90) (end 124 90) (stroke (width 0.1) (type default)) (layer "Edge.Cuts"))
 (gr_arc (start 129 102) (mid 127.828427 104.828427) (end 125 106) (stroke (width 0.1) (type default)) (layer "Edge.Cuts"))
 (gr_line (start 125 106) (end 112 106) (stroke (width 0.1) (type default)) (layer "Edge.Cuts"))
 (gr_arc (start 108 94) (mid 109.171573 91.171573) (end 112 90) (stroke (width 0.1) (type default)) (layer "Edge.Cuts"))
 (gr_arc (start 112 106) (mid 109.171573 104.828427) (end 108 102) (stroke (width 0.1) (type default)) (layer "Edge.Cuts"))
 (segment (start 116.98 104) (end 116.84 104.14) (width 0.25) (layer "F.Cu") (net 3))
 (segment (start 119 104) (end 116.98 104) (width 0.25) (layer "F.Cu") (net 3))
 (via (at 116.84 104.14) (size 0.8) (drill 0.4) (layers "F.Cu" "B.Cu") (free) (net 3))
 (segment (start 119 99.825) (end 119 102.4) (width 0.25) (layer "F.Cu") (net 4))
 (segment (start 124.968 98.044) (end 119.044 98.044) (width 0.25) (layer "F.Cu") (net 2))
 (segment (start 126.212 96.8) (end 124.968 98.044) (width 0.25) (layer "F.Cu") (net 2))
 (segment (start 119.044 98.044) (end 119 98) (width 0.25) (layer "F.Cu") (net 2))
 (segment (start 126.212 93.98) (end 126.212 96.8) (width 0.25) (layer "F.Cu") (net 2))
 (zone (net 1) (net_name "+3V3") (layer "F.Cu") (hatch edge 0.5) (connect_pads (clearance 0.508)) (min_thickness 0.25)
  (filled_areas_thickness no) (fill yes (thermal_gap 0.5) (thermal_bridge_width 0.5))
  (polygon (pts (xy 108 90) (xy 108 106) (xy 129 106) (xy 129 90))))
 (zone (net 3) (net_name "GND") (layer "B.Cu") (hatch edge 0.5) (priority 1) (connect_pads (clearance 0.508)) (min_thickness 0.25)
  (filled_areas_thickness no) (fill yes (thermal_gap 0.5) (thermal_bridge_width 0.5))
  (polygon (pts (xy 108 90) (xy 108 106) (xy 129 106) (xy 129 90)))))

